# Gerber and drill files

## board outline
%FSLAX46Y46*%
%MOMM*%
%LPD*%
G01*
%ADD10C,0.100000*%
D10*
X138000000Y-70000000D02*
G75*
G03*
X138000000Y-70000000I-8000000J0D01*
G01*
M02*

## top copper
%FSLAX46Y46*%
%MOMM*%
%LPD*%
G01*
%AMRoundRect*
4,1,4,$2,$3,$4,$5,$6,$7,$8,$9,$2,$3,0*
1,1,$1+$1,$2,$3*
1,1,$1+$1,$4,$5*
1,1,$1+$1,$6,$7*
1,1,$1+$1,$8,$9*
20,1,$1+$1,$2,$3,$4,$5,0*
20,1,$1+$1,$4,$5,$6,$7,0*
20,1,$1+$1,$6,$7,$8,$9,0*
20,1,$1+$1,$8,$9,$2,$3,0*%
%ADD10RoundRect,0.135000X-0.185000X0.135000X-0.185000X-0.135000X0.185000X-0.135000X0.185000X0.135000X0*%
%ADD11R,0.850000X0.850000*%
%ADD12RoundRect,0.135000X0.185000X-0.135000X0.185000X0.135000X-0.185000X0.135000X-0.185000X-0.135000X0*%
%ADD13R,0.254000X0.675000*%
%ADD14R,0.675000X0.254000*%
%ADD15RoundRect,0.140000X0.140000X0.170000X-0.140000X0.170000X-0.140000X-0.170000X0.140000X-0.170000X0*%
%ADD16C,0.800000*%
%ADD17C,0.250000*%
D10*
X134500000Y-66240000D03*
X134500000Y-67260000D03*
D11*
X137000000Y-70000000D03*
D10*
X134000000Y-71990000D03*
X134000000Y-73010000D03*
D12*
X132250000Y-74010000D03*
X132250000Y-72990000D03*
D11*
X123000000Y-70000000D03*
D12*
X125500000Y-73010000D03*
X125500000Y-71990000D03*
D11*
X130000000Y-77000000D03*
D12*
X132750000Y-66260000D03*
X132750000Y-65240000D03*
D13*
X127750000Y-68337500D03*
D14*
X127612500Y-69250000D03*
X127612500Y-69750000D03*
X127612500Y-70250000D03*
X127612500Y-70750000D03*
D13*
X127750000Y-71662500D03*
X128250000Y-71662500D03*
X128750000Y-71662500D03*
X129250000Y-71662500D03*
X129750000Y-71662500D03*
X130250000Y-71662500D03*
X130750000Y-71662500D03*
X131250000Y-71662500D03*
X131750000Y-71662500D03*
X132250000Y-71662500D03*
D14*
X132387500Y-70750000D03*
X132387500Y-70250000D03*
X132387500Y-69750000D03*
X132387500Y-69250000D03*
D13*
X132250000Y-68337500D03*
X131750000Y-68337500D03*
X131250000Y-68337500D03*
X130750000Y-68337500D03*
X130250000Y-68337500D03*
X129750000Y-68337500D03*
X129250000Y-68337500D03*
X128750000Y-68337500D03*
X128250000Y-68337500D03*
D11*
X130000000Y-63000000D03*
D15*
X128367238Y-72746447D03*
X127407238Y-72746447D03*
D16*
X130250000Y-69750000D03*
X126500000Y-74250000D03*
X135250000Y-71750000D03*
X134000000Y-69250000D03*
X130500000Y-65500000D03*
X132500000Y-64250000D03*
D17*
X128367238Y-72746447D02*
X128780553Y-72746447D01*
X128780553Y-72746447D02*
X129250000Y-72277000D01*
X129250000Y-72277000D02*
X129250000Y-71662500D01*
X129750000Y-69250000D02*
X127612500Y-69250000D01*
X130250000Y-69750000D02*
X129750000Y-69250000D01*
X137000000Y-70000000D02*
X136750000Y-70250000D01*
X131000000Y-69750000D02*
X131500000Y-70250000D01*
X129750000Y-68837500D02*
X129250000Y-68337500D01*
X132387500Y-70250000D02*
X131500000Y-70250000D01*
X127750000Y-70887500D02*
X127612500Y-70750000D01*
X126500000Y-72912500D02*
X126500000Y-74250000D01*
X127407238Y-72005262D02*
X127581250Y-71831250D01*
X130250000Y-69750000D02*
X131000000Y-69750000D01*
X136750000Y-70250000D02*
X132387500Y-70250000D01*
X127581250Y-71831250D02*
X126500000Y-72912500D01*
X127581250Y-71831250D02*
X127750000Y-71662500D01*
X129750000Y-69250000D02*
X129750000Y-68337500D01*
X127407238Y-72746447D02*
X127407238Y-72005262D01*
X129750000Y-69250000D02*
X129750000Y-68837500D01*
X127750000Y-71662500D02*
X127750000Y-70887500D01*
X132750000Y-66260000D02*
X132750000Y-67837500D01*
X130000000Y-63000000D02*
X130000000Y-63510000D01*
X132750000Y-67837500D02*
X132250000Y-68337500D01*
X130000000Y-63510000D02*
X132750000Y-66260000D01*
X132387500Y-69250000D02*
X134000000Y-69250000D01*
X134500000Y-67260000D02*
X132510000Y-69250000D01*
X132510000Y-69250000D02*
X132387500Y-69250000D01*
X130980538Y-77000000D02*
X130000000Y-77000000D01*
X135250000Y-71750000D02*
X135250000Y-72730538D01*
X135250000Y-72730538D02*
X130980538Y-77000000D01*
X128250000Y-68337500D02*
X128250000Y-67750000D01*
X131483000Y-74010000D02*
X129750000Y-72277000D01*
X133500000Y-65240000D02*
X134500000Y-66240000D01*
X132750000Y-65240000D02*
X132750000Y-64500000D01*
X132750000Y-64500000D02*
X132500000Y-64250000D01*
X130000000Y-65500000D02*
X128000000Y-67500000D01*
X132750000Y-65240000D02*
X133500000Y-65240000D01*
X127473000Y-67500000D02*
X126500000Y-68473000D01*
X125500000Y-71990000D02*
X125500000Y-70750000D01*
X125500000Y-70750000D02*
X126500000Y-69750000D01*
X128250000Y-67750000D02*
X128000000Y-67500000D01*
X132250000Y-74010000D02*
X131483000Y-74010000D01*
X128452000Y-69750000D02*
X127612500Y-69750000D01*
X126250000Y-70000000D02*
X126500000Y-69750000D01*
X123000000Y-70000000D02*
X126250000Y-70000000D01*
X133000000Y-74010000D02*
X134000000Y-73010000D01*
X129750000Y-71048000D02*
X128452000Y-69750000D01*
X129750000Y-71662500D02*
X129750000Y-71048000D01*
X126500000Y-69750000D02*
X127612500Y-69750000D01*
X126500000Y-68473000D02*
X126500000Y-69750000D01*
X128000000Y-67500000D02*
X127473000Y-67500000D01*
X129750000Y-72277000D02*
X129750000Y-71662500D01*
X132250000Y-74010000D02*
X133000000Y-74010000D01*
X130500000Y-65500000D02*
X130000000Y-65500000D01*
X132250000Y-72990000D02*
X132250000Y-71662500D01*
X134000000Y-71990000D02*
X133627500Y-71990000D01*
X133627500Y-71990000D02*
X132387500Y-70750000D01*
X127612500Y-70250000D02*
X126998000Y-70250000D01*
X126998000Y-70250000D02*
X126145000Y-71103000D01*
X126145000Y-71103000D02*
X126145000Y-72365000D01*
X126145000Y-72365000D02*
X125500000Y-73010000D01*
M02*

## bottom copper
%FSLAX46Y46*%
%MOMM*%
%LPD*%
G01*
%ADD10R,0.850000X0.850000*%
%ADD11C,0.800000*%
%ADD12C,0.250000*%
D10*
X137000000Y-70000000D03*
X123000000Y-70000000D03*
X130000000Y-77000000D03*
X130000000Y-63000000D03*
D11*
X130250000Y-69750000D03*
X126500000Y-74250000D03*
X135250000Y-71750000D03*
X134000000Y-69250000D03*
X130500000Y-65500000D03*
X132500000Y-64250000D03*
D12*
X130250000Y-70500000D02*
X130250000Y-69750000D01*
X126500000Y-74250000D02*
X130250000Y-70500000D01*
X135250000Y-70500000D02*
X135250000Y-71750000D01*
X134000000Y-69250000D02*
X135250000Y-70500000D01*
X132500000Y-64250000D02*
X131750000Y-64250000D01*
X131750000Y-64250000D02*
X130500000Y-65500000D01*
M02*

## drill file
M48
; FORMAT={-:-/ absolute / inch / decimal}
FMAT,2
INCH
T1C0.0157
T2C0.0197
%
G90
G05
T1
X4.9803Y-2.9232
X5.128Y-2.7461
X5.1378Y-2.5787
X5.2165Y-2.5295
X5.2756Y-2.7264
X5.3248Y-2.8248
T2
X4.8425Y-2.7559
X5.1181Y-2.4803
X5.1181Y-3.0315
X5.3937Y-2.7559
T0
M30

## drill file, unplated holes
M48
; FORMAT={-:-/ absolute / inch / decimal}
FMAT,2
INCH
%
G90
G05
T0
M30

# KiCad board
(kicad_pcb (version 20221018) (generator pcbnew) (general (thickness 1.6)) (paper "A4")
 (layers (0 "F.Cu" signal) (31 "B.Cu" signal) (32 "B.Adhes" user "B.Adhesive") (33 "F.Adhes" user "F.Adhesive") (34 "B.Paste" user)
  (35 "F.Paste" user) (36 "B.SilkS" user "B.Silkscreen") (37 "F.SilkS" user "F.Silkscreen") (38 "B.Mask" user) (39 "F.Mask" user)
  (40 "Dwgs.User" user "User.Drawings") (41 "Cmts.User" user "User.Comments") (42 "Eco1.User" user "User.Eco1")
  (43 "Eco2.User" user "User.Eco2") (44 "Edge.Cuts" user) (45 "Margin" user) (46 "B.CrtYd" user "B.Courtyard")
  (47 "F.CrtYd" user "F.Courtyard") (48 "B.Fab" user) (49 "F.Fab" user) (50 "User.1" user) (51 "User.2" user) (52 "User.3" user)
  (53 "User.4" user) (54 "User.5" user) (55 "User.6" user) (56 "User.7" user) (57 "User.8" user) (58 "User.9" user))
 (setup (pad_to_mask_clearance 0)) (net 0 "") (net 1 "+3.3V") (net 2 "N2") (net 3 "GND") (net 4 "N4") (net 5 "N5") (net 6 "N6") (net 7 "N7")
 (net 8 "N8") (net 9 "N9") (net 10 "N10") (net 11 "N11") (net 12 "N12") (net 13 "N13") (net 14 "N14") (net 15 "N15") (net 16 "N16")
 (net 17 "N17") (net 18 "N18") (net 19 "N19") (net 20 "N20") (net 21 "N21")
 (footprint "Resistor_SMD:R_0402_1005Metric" (layer "F.Cu") (at 134.5 66.75 -90)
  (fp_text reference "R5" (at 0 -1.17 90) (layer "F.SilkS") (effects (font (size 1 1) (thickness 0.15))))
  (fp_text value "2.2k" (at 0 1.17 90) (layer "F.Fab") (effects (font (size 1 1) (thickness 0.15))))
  (pad "1" smd roundrect (at -0.51 0 270) (size 0.54 0.64) (layers "F.Cu" "F.Paste" "F.Mask") (roundrect_rratio 0.25) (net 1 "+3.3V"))
  (pad "2" smd roundrect (at 0.51 0 270) (size 0.54 0.64) (layers "F.Cu" "F.Paste" "F.Mask") (roundrect_rratio 0.25) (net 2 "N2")))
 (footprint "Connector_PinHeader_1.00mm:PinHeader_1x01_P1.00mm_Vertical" (layer "F.Cu") (at 137 70 -90)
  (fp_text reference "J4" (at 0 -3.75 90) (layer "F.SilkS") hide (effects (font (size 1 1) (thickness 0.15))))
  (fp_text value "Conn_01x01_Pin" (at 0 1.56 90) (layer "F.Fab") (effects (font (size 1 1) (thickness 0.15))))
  (pad "1" thru_hole rect (at 0 0 270) (size 0.85 0.85) (drill 0.5) (layers "*.Cu" "*.Mask") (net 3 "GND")))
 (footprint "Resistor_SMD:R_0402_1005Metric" (layer "F.Cu") (at 134 72.5 -90)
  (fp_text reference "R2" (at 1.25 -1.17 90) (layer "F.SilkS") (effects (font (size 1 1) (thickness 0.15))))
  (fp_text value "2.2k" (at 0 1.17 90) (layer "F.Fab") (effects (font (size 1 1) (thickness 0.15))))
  (pad "1" smd roundrect (at -0.51 0 270) (size 0.54 0.64) (layers "F.Cu" "F.Paste" "F.Mask") (roundrect_rratio 0.25) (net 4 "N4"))
  (pad "2" smd roundrect (at 0.51 0 270) (size 0.54 0.64) (layers "F.Cu" "F.Paste" "F.Mask") (roundrect_rratio 0.25) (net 1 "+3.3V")))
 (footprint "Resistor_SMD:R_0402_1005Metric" (layer "F.Cu") (at 132.25 73.5 90)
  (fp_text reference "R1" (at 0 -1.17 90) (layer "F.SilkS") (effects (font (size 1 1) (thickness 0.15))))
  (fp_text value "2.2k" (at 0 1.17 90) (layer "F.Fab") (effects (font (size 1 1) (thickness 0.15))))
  (pad "1" smd roundrect (at -0.51 0 90) (size 0.54 0.64) (layers "F.Cu" "F.Paste" "F.Mask") (roundrect_rratio 0.25) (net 1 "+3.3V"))
  (pad "2" smd roundrect (at 0.51 0 90) (size 0.54 0.64) (layers "F.Cu" "F.Paste" "F.Mask") (roundrect_rratio 0.25) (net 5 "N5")))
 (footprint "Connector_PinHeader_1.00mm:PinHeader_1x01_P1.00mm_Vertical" (layer "F.Cu") (at 123 70 90)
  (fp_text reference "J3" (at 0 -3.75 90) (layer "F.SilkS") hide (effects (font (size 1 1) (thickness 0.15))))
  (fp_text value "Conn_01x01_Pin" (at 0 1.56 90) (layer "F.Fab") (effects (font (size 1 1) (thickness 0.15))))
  (pad "1" thru_hole rect (at 0 0 90) (size 0.85 0.85) (drill 0.5) (layers "*.Cu" "*.Mask") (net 1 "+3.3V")))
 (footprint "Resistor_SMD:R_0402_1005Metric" (layer "F.Cu") (at 125.5 72.5 90)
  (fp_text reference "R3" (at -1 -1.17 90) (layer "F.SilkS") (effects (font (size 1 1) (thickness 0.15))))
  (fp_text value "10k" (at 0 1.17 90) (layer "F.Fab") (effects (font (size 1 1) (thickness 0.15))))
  (pad "1" smd roundrect (at -0.51 0 90) (size 0.54 0.64) (layers "F.Cu" "F.Paste" "F.Mask") (roundrect_rratio 0.25) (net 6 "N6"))
  (pad "2" smd roundrect (at 0.51 0 90) (size 0.54 0.64) (layers "F.Cu" "F.Paste" "F.Mask") (roundrect_rratio 0.25) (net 1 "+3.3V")))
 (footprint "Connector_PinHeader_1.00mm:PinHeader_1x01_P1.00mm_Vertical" (layer "F.Cu") (at 130 77 180)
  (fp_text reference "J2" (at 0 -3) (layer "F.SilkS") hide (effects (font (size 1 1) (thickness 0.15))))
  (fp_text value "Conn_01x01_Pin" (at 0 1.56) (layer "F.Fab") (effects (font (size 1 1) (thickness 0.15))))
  (pad "1" thru_hole rect (at 0 0 180) (size 0.85 0.85) (drill 0.5) (layers "*.Cu" "*.Mask") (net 2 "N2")))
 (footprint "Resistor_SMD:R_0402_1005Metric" (layer "F.Cu") (at 132.75 65.75 90)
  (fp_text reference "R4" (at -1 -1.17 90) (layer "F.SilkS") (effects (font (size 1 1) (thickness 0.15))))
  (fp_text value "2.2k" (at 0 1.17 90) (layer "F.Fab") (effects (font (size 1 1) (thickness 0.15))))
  (pad "1" smd roundrect (at -0.51 0 90) (size 0.54 0.64) (layers "F.Cu" "F.Paste" "F.Mask") (roundrect_rratio 0.25) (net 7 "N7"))
  (pad "2" smd roundrect (at 0.51 0 90) (size 0.54 0.64) (layers "F.Cu" "F.Paste" "F.Mask") (roundrect_rratio 0.25) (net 1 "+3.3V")))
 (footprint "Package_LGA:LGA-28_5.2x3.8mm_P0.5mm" (layer "F.Cu") (at 130 70)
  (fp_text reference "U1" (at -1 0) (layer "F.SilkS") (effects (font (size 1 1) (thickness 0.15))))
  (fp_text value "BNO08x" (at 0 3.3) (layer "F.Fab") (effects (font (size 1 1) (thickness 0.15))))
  (pad "1" smd rect (at -2.25 -1.6625) (size 0.254 0.675) (layers "F.Cu" "F.Paste" "F.Mask") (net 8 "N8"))
  (pad "2" smd rect (at -2.3875 -0.75 90) (size 0.254 0.675) (layers "F.Cu" "F.Paste" "F.Mask") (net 3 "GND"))
  (pad "3" smd rect (at -2.3875 -0.25 90) (size 0.254 0.675) (layers "F.Cu" "F.Paste" "F.Mask") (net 1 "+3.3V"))
  (pad "4" smd rect (at -2.3875 0.25 90) (size 0.254 0.675) (layers "F.Cu" "F.Paste" "F.Mask") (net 6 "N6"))
  (pad "5" smd rect (at -2.3875 0.75 90) (size 0.254 0.675) (layers "F.Cu" "F.Paste" "F.Mask") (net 3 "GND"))
  (pad "6" smd rect (at -2.25 1.6625) (size 0.254 0.675) (layers "F.Cu" "F.Paste" "F.Mask") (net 3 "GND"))
  (pad "7" smd rect (at -1.75 1.6625) (size 0.254 0.675) (layers "F.Cu" "F.Paste" "F.Mask") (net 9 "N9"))
  (pad "8" smd rect (at -1.25 1.6625) (size 0.254 0.675) (layers "F.Cu" "F.Paste" "F.Mask") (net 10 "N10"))
  (pad "9" smd rect (at -0.75 1.6625) (size 0.254 0.675) (layers "F.Cu" "F.Paste" "F.Mask") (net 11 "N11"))
  (pad "10" smd rect (at -0.25 1.6625) (size 0.254 0.675) (layers "F.Cu" "F.Paste" "F.Mask") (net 1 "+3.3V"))
  (pad "11" smd rect (at 0.25 1.6625) (size 0.254 0.675) (layers "F.Cu" "F.Paste" "F.Mask") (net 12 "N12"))
  (pad "12" smd rect (at 0.75 1.6625) (size 0.254 0.675) (layers "F.Cu" "F.Paste" "F.Mask") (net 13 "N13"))
  (pad "13" smd rect (at 1.25 1.6625) (size 0.254 0.675) (layers "F.Cu" "F.Paste" "F.Mask") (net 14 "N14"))
  (pad "14" smd rect (at 1.75 1.6625) (size 0.254 0.675) (layers "F.Cu" "F.Paste" "F.Mask") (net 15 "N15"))
  (pad "15" smd rect (at 2.25 1.6625) (size 0.254 0.675) (layers "F.Cu" "F.Paste" "F.Mask") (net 5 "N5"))
  (pad "16" smd rect (at 2.3875 0.75 90) (size 0.254 0.675) (layers "F.Cu" "F.Paste" "F.Mask") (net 4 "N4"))
  (pad "17" smd rect (at 2.3875 0.25 90) (size 0.254 0.675) (layers "F.Cu" "F.Paste" "F.Mask") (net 3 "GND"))
  (pad "18" smd rect (at 2.3875 -0.25 90) (size 0.254 0.675) (layers "F.Cu" "F.Paste" "F.Mask") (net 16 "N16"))
  (pad "19" smd rect (at 2.3875 -0.75 90) (size 0.254 0.675) (layers "F.Cu" "F.Paste" "F.Mask") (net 2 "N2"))
  (pad "20" smd rect (at 2.25 -1.6625) (size 0.254 0.675) (layers "F.Cu" "F.Paste" "F.Mask") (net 7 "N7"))
  (pad "21" smd rect (at 1.75 -1.6625) (size 0.254 0.675) (layers "F.Cu" "F.Paste" "F.Mask") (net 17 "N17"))
  (pad "22" smd rect (at 1.25 -1.6625) (size 0.254 0.675) (layers "F.Cu" "F.Paste" "F.Mask") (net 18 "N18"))
  (pad "23" smd rect (at 0.75 -1.6625) (size 0.254 0.675) (layers "F.Cu" "F.Paste" "F.Mask") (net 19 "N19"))
  (pad "24" smd rect (at 0.25 -1.6625) (size 0.254 0.675) (layers "F.Cu" "F.Paste" "F.Mask") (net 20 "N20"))
  (pad "25" smd rect (at -0.25 -1.6625) (size 0.254 0.675) (layers "F.Cu" "F.Paste" "F.Mask") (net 3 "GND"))
  (pad "26" smd rect (at -0.75 -1.6625) (size 0.254 0.675) (layers "F.Cu" "F.Paste" "F.Mask") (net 3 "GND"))
  (pad "27" smd rect (at -1.25 -1.6625) (size 0.254 0.675) (layers "F.Cu" "F.Paste" "F.Mask") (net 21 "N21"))
  (pad "28" smd rect (at -1.75 -1.6625) (size 0.254 0.675) (layers "F.Cu" "F.Paste" "F.Mask") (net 1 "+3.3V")))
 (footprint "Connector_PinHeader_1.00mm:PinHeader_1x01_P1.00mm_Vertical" (layer "F.Cu") (at 130 63)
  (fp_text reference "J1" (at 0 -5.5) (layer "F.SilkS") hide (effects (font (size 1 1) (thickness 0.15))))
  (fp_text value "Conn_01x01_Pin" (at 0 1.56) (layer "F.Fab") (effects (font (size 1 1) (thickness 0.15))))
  (pad "1" thru_hole rect (at 0 0) (size 0.85 0.85) (drill 0.5) (layers "*.Cu" "*.Mask") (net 7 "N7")))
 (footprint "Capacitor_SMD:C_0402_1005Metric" (layer "F.Cu") (at 127.887238 72.746447 180)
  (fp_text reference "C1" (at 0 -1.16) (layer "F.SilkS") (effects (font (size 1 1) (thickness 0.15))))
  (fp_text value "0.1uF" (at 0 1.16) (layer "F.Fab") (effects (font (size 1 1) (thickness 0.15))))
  (pad "1" smd roundrect (at -0.48 0 180) (size 0.56 0.62) (layers "F.Cu" "F.Paste" "F.Mask") (roundrect_rratio 0.25) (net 11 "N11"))
  (pad "2" smd roundrect (at 0.48 0 180) (size 0.56 0.62) (layers "F.Cu" "F.Paste" "F.Mask") (roundrect_rratio 0.25) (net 3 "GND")))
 (gr_circle (center 130 70) (end 138 70) (stroke (width 0.1) (type default)) (fill none) (layer "Edge.Cuts"))
 (segment (start 128.367238 72.746447) (end 128.780553 72.746447) (width 0.25) (layer "F.Cu") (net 11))
 (segment (start 128.780553 72.746447) (end 129.25 72.277) (width 0.25) (layer "F.Cu") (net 11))
 (segment (start 129.25 72.277) (end 129.25 71.6625) (width 0.25) (layer "F.Cu") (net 11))
 (segment (start 129.75 69.25) (end 127.6125 69.25) (width 0.25) (layer "F.Cu") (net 3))
 (segment (start 130.25 69.75) (end 129.75 69.25) (width 0.25) (layer "F.Cu") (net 3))
 (segment (start 137 70) (end 136.75 70.25) (width 0.25) (layer "F.Cu") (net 3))
 (segment (start 131 69.75) (end 131.5 70.25) (width 0.25) (layer "F.Cu") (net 3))
 (segment (start 129.75 68.8375) (end 129.25 68.3375) (width 0.25) (layer "F.Cu") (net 3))
 (segment (start 132.3875 70.25) (end 131.5 70.25) (width 0.25) (layer "F.Cu") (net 3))
 (segment (start 127.75 70.8875) (end 127.6125 70.75) (width 0.25) (layer "F.Cu") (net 3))
 (segment (start 126.5 72.9125) (end 126.5 74.25) (width 0.25) (layer "F.Cu") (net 3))
 (segment (start 127.407238 72.005262) (end 127.58125 71.83125) (width 0.25) (layer "F.Cu") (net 3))
 (segment (start 130.25 69.75) (end 131 69.75) (width 0.25) (layer "F.Cu") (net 3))
 (segment (start 136.75 70.25) (end 132.3875 70.25) (width 0.25) (layer "F.Cu") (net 3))
 (segment (start 127.58125 71.83125) (end 126.5 72.9125) (width 0.25) (layer "F.Cu") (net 3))
 (segment (start 127.58125 71.83125) (end 127.75 71.6625) (width 0.25) (layer "F.Cu") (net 3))
 (segment (start 129.75 69.25) (end 129.75 68.3375) (width 0.25) (layer "F.Cu") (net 3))
 (segment (start 127.407238 72.746447) (end 127.407238 72.005262) (width 0.25) (layer "F.Cu") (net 3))
 (segment (start 129.75 69.25) (end 129.75 68.8375) (width 0.25) (layer "F.Cu") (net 3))
 (segment (start 127.75 71.6625) (end 127.75 70.8875) (width 0.25) (layer "F.Cu") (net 3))
 (via (at 130.25 69.75) (size 0.8) (drill 0.4) (layers "F.Cu" "B.Cu") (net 3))
 (via (at 126.5 74.25) (size 0.8) (drill 0.4) (layers "F.Cu" "B.Cu") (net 3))
 (segment (start 130.25 70.5) (end 130.25 69.75) (width 0.25) (layer "B.Cu") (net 3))
 (segment (start 126.5 74.25) (end 130.25 70.5) (width 0.25) (layer "B.Cu") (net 3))
 (segment (start 132.75 66.26) (end 132.75 67.8375) (width 0.25) (layer "F.Cu") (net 7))
 (segment (start 130 63) (end 130 63.51) (width 0.25) (layer "F.Cu") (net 7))
 (segment (start 132.75 67.8375) (end 132.25 68.3375) (width 0.25) (layer "F.Cu") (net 7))
 (segment (start 130 63.51) (end 132.75 66.26) (width 0.25) (layer "F.Cu") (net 7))
 (segment (start 132.3875 69.25) (end 134 69.25) (width 0.25) (layer "F.Cu") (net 2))
 (segment (start 134.5 67.26) (end 132.51 69.25) (width 0.25) (layer "F.Cu") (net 2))
 (segment (start 132.51 69.25) (end 132.3875 69.25) (width 0.25) (layer "F.Cu") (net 2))
 (segment (start 130.980538 77) (end 130 77) (width 0.25) (layer "F.Cu") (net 2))
 (segment (start 135.25 71.75) (end 135.25 72.730538) (width 0.25) (layer "F.Cu") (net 2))
 (segment (start 135.25 72.730538) (end 130.980538 77) (width 0.25) (layer "F.Cu") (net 2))
 (via (at 135.25 71.75) (size 0.8) (drill 0.4) (layers "F.Cu" "B.Cu") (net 2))
 (via (at 134 69.25) (size 0.8) (drill 0.4) (layers "F.Cu" "B.Cu") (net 2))
 (segment (start 135.25 70.5) (end 135.25 71.75) (width 0.25) (layer "B.Cu") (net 2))
 (segment (start 134 69.25) (end 135.25 70.5) (width 0.25) (layer "B.Cu") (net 2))
 (segment (start 128.25 68.3375) (end 128.25 67.75) (width 0.25) (layer "F.Cu") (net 1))
 (segment (start 131.483 74.01) (end 129.75 72.277) (width 0.25) (layer "F.Cu") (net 1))
 (segment (start 133.5 65.24) (end 134.5 66.24) (width 0.25) (layer "F.Cu") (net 1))
 (segment (start 132.75 65.24) (end 132.75 64.5) (width 0.25) (layer "F.Cu") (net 1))
 (segment (start 132.75 64.5) (end 132.5 64.25) (width 0.25) (layer "F.Cu") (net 1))
 (segment (start 130 65.5) (end 128 67.5) (width 0.25) (layer "F.Cu") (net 1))
 (segment (start 132.75 65.24) (end 133.5 65.24) (width 0.25) (layer "F.Cu") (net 1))
 (segment (start 127.473 67.5) (end 126.5 68.473) (width 0.25) (layer "F.Cu") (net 1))
 (segment (start 125.5 71.99) (end 125.5 70.75) (width 0.25) (layer "F.Cu") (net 1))
 (segment (start 125.5 70.75) (end 126.5 69.75) (width 0.25) (layer "F.Cu") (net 1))
 (segment (start 128.25 67.75) (end 128 67.5) (width 0.25) (layer "F.Cu") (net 1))
 (segment (start 132.25 74.01) (end 131.483 74.01) (width 0.25) (layer "F.Cu") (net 1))
 (segment (start 128.452 69.75) (end 127.6125 69.75) (width 0.25) (layer "F.Cu") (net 1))
 (segment (start 126.25 70) (end 126.5 69.75) (width 0.25) (layer "F.Cu") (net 1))
 (segment (start 123 70) (end 126.25 70) (width 0.25) (layer "F.Cu") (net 1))
 (segment (start 133 74.01) (end 134 73.01) (width 0.25) (layer "F.Cu") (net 1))
 (segment (start 129.75 71.048) (end 128.452 69.75) (width 0.25) (layer "F.Cu") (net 1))
 (segment (start 129.75 71.6625) (end 129.75 71.048) (width 0.25) (layer "F.Cu") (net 1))
 (segment (start 126.5 69.75) (end 127.6125 69.75) (width 0.25) (layer "F.Cu") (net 1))
 (segment (start 126.5 68.473) (end 126.5 69.75) (width 0.25) (layer "F.Cu") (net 1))
 (segment (start 128 67.5) (end 127.473 67.5) (width 0.25) (layer "F.Cu") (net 1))
 (segment (start 129.75 72.277) (end 129.75 71.6625) (width 0.25) (layer "F.Cu") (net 1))
 (segment (start 132.25 74.01) (end 133 74.01) (width 0.25) (layer "F.Cu") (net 1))
 (segment (start 130.5 65.5) (end 130 65.5) (width 0.25) (layer "F.Cu") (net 1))
 (via (at 130.5 65.5) (size 0.8) (drill 0.4) (layers "F.Cu" "B.Cu") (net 1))
 (via (at 132.5 64.25) (size 0.8) (drill 0.4) (layers "F.Cu" "B.Cu") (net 1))
 (segment (start 132.5 64.25) (end 131.75 64.25) (width 0.25) (layer "B.Cu") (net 1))
 (segment (start 131.75 64.25) (end 130.5 65.5) (width 0.25) (layer "B.Cu") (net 1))
 (segment (start 132.25 72.99) (end 132.25 71.6625) (width 0.25) (layer "F.Cu") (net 5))
 (segment (start 134 71.99) (end 133.6275 71.99) (width 0.25) (layer "F.Cu") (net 4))
 (segment (start 133.6275 71.99) (end 132.3875 70.75) (width 0.25) (layer "F.Cu") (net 4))
 (segment (start 127.6125 70.25) (end 126.998 70.25) (width 0.25) (layer "F.Cu") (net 6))
 (segment (start 126.998 70.25) (end 126.145 71.103) (width 0.25) (layer "F.Cu") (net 6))
 (segment (start 126.145 71.103) (end 126.145 72.365) (width 0.25) (layer "F.Cu") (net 6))
 (segment (start 126.145 72.365) (end 125.5 73.01) (width 0.25) (layer "F.Cu") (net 6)))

